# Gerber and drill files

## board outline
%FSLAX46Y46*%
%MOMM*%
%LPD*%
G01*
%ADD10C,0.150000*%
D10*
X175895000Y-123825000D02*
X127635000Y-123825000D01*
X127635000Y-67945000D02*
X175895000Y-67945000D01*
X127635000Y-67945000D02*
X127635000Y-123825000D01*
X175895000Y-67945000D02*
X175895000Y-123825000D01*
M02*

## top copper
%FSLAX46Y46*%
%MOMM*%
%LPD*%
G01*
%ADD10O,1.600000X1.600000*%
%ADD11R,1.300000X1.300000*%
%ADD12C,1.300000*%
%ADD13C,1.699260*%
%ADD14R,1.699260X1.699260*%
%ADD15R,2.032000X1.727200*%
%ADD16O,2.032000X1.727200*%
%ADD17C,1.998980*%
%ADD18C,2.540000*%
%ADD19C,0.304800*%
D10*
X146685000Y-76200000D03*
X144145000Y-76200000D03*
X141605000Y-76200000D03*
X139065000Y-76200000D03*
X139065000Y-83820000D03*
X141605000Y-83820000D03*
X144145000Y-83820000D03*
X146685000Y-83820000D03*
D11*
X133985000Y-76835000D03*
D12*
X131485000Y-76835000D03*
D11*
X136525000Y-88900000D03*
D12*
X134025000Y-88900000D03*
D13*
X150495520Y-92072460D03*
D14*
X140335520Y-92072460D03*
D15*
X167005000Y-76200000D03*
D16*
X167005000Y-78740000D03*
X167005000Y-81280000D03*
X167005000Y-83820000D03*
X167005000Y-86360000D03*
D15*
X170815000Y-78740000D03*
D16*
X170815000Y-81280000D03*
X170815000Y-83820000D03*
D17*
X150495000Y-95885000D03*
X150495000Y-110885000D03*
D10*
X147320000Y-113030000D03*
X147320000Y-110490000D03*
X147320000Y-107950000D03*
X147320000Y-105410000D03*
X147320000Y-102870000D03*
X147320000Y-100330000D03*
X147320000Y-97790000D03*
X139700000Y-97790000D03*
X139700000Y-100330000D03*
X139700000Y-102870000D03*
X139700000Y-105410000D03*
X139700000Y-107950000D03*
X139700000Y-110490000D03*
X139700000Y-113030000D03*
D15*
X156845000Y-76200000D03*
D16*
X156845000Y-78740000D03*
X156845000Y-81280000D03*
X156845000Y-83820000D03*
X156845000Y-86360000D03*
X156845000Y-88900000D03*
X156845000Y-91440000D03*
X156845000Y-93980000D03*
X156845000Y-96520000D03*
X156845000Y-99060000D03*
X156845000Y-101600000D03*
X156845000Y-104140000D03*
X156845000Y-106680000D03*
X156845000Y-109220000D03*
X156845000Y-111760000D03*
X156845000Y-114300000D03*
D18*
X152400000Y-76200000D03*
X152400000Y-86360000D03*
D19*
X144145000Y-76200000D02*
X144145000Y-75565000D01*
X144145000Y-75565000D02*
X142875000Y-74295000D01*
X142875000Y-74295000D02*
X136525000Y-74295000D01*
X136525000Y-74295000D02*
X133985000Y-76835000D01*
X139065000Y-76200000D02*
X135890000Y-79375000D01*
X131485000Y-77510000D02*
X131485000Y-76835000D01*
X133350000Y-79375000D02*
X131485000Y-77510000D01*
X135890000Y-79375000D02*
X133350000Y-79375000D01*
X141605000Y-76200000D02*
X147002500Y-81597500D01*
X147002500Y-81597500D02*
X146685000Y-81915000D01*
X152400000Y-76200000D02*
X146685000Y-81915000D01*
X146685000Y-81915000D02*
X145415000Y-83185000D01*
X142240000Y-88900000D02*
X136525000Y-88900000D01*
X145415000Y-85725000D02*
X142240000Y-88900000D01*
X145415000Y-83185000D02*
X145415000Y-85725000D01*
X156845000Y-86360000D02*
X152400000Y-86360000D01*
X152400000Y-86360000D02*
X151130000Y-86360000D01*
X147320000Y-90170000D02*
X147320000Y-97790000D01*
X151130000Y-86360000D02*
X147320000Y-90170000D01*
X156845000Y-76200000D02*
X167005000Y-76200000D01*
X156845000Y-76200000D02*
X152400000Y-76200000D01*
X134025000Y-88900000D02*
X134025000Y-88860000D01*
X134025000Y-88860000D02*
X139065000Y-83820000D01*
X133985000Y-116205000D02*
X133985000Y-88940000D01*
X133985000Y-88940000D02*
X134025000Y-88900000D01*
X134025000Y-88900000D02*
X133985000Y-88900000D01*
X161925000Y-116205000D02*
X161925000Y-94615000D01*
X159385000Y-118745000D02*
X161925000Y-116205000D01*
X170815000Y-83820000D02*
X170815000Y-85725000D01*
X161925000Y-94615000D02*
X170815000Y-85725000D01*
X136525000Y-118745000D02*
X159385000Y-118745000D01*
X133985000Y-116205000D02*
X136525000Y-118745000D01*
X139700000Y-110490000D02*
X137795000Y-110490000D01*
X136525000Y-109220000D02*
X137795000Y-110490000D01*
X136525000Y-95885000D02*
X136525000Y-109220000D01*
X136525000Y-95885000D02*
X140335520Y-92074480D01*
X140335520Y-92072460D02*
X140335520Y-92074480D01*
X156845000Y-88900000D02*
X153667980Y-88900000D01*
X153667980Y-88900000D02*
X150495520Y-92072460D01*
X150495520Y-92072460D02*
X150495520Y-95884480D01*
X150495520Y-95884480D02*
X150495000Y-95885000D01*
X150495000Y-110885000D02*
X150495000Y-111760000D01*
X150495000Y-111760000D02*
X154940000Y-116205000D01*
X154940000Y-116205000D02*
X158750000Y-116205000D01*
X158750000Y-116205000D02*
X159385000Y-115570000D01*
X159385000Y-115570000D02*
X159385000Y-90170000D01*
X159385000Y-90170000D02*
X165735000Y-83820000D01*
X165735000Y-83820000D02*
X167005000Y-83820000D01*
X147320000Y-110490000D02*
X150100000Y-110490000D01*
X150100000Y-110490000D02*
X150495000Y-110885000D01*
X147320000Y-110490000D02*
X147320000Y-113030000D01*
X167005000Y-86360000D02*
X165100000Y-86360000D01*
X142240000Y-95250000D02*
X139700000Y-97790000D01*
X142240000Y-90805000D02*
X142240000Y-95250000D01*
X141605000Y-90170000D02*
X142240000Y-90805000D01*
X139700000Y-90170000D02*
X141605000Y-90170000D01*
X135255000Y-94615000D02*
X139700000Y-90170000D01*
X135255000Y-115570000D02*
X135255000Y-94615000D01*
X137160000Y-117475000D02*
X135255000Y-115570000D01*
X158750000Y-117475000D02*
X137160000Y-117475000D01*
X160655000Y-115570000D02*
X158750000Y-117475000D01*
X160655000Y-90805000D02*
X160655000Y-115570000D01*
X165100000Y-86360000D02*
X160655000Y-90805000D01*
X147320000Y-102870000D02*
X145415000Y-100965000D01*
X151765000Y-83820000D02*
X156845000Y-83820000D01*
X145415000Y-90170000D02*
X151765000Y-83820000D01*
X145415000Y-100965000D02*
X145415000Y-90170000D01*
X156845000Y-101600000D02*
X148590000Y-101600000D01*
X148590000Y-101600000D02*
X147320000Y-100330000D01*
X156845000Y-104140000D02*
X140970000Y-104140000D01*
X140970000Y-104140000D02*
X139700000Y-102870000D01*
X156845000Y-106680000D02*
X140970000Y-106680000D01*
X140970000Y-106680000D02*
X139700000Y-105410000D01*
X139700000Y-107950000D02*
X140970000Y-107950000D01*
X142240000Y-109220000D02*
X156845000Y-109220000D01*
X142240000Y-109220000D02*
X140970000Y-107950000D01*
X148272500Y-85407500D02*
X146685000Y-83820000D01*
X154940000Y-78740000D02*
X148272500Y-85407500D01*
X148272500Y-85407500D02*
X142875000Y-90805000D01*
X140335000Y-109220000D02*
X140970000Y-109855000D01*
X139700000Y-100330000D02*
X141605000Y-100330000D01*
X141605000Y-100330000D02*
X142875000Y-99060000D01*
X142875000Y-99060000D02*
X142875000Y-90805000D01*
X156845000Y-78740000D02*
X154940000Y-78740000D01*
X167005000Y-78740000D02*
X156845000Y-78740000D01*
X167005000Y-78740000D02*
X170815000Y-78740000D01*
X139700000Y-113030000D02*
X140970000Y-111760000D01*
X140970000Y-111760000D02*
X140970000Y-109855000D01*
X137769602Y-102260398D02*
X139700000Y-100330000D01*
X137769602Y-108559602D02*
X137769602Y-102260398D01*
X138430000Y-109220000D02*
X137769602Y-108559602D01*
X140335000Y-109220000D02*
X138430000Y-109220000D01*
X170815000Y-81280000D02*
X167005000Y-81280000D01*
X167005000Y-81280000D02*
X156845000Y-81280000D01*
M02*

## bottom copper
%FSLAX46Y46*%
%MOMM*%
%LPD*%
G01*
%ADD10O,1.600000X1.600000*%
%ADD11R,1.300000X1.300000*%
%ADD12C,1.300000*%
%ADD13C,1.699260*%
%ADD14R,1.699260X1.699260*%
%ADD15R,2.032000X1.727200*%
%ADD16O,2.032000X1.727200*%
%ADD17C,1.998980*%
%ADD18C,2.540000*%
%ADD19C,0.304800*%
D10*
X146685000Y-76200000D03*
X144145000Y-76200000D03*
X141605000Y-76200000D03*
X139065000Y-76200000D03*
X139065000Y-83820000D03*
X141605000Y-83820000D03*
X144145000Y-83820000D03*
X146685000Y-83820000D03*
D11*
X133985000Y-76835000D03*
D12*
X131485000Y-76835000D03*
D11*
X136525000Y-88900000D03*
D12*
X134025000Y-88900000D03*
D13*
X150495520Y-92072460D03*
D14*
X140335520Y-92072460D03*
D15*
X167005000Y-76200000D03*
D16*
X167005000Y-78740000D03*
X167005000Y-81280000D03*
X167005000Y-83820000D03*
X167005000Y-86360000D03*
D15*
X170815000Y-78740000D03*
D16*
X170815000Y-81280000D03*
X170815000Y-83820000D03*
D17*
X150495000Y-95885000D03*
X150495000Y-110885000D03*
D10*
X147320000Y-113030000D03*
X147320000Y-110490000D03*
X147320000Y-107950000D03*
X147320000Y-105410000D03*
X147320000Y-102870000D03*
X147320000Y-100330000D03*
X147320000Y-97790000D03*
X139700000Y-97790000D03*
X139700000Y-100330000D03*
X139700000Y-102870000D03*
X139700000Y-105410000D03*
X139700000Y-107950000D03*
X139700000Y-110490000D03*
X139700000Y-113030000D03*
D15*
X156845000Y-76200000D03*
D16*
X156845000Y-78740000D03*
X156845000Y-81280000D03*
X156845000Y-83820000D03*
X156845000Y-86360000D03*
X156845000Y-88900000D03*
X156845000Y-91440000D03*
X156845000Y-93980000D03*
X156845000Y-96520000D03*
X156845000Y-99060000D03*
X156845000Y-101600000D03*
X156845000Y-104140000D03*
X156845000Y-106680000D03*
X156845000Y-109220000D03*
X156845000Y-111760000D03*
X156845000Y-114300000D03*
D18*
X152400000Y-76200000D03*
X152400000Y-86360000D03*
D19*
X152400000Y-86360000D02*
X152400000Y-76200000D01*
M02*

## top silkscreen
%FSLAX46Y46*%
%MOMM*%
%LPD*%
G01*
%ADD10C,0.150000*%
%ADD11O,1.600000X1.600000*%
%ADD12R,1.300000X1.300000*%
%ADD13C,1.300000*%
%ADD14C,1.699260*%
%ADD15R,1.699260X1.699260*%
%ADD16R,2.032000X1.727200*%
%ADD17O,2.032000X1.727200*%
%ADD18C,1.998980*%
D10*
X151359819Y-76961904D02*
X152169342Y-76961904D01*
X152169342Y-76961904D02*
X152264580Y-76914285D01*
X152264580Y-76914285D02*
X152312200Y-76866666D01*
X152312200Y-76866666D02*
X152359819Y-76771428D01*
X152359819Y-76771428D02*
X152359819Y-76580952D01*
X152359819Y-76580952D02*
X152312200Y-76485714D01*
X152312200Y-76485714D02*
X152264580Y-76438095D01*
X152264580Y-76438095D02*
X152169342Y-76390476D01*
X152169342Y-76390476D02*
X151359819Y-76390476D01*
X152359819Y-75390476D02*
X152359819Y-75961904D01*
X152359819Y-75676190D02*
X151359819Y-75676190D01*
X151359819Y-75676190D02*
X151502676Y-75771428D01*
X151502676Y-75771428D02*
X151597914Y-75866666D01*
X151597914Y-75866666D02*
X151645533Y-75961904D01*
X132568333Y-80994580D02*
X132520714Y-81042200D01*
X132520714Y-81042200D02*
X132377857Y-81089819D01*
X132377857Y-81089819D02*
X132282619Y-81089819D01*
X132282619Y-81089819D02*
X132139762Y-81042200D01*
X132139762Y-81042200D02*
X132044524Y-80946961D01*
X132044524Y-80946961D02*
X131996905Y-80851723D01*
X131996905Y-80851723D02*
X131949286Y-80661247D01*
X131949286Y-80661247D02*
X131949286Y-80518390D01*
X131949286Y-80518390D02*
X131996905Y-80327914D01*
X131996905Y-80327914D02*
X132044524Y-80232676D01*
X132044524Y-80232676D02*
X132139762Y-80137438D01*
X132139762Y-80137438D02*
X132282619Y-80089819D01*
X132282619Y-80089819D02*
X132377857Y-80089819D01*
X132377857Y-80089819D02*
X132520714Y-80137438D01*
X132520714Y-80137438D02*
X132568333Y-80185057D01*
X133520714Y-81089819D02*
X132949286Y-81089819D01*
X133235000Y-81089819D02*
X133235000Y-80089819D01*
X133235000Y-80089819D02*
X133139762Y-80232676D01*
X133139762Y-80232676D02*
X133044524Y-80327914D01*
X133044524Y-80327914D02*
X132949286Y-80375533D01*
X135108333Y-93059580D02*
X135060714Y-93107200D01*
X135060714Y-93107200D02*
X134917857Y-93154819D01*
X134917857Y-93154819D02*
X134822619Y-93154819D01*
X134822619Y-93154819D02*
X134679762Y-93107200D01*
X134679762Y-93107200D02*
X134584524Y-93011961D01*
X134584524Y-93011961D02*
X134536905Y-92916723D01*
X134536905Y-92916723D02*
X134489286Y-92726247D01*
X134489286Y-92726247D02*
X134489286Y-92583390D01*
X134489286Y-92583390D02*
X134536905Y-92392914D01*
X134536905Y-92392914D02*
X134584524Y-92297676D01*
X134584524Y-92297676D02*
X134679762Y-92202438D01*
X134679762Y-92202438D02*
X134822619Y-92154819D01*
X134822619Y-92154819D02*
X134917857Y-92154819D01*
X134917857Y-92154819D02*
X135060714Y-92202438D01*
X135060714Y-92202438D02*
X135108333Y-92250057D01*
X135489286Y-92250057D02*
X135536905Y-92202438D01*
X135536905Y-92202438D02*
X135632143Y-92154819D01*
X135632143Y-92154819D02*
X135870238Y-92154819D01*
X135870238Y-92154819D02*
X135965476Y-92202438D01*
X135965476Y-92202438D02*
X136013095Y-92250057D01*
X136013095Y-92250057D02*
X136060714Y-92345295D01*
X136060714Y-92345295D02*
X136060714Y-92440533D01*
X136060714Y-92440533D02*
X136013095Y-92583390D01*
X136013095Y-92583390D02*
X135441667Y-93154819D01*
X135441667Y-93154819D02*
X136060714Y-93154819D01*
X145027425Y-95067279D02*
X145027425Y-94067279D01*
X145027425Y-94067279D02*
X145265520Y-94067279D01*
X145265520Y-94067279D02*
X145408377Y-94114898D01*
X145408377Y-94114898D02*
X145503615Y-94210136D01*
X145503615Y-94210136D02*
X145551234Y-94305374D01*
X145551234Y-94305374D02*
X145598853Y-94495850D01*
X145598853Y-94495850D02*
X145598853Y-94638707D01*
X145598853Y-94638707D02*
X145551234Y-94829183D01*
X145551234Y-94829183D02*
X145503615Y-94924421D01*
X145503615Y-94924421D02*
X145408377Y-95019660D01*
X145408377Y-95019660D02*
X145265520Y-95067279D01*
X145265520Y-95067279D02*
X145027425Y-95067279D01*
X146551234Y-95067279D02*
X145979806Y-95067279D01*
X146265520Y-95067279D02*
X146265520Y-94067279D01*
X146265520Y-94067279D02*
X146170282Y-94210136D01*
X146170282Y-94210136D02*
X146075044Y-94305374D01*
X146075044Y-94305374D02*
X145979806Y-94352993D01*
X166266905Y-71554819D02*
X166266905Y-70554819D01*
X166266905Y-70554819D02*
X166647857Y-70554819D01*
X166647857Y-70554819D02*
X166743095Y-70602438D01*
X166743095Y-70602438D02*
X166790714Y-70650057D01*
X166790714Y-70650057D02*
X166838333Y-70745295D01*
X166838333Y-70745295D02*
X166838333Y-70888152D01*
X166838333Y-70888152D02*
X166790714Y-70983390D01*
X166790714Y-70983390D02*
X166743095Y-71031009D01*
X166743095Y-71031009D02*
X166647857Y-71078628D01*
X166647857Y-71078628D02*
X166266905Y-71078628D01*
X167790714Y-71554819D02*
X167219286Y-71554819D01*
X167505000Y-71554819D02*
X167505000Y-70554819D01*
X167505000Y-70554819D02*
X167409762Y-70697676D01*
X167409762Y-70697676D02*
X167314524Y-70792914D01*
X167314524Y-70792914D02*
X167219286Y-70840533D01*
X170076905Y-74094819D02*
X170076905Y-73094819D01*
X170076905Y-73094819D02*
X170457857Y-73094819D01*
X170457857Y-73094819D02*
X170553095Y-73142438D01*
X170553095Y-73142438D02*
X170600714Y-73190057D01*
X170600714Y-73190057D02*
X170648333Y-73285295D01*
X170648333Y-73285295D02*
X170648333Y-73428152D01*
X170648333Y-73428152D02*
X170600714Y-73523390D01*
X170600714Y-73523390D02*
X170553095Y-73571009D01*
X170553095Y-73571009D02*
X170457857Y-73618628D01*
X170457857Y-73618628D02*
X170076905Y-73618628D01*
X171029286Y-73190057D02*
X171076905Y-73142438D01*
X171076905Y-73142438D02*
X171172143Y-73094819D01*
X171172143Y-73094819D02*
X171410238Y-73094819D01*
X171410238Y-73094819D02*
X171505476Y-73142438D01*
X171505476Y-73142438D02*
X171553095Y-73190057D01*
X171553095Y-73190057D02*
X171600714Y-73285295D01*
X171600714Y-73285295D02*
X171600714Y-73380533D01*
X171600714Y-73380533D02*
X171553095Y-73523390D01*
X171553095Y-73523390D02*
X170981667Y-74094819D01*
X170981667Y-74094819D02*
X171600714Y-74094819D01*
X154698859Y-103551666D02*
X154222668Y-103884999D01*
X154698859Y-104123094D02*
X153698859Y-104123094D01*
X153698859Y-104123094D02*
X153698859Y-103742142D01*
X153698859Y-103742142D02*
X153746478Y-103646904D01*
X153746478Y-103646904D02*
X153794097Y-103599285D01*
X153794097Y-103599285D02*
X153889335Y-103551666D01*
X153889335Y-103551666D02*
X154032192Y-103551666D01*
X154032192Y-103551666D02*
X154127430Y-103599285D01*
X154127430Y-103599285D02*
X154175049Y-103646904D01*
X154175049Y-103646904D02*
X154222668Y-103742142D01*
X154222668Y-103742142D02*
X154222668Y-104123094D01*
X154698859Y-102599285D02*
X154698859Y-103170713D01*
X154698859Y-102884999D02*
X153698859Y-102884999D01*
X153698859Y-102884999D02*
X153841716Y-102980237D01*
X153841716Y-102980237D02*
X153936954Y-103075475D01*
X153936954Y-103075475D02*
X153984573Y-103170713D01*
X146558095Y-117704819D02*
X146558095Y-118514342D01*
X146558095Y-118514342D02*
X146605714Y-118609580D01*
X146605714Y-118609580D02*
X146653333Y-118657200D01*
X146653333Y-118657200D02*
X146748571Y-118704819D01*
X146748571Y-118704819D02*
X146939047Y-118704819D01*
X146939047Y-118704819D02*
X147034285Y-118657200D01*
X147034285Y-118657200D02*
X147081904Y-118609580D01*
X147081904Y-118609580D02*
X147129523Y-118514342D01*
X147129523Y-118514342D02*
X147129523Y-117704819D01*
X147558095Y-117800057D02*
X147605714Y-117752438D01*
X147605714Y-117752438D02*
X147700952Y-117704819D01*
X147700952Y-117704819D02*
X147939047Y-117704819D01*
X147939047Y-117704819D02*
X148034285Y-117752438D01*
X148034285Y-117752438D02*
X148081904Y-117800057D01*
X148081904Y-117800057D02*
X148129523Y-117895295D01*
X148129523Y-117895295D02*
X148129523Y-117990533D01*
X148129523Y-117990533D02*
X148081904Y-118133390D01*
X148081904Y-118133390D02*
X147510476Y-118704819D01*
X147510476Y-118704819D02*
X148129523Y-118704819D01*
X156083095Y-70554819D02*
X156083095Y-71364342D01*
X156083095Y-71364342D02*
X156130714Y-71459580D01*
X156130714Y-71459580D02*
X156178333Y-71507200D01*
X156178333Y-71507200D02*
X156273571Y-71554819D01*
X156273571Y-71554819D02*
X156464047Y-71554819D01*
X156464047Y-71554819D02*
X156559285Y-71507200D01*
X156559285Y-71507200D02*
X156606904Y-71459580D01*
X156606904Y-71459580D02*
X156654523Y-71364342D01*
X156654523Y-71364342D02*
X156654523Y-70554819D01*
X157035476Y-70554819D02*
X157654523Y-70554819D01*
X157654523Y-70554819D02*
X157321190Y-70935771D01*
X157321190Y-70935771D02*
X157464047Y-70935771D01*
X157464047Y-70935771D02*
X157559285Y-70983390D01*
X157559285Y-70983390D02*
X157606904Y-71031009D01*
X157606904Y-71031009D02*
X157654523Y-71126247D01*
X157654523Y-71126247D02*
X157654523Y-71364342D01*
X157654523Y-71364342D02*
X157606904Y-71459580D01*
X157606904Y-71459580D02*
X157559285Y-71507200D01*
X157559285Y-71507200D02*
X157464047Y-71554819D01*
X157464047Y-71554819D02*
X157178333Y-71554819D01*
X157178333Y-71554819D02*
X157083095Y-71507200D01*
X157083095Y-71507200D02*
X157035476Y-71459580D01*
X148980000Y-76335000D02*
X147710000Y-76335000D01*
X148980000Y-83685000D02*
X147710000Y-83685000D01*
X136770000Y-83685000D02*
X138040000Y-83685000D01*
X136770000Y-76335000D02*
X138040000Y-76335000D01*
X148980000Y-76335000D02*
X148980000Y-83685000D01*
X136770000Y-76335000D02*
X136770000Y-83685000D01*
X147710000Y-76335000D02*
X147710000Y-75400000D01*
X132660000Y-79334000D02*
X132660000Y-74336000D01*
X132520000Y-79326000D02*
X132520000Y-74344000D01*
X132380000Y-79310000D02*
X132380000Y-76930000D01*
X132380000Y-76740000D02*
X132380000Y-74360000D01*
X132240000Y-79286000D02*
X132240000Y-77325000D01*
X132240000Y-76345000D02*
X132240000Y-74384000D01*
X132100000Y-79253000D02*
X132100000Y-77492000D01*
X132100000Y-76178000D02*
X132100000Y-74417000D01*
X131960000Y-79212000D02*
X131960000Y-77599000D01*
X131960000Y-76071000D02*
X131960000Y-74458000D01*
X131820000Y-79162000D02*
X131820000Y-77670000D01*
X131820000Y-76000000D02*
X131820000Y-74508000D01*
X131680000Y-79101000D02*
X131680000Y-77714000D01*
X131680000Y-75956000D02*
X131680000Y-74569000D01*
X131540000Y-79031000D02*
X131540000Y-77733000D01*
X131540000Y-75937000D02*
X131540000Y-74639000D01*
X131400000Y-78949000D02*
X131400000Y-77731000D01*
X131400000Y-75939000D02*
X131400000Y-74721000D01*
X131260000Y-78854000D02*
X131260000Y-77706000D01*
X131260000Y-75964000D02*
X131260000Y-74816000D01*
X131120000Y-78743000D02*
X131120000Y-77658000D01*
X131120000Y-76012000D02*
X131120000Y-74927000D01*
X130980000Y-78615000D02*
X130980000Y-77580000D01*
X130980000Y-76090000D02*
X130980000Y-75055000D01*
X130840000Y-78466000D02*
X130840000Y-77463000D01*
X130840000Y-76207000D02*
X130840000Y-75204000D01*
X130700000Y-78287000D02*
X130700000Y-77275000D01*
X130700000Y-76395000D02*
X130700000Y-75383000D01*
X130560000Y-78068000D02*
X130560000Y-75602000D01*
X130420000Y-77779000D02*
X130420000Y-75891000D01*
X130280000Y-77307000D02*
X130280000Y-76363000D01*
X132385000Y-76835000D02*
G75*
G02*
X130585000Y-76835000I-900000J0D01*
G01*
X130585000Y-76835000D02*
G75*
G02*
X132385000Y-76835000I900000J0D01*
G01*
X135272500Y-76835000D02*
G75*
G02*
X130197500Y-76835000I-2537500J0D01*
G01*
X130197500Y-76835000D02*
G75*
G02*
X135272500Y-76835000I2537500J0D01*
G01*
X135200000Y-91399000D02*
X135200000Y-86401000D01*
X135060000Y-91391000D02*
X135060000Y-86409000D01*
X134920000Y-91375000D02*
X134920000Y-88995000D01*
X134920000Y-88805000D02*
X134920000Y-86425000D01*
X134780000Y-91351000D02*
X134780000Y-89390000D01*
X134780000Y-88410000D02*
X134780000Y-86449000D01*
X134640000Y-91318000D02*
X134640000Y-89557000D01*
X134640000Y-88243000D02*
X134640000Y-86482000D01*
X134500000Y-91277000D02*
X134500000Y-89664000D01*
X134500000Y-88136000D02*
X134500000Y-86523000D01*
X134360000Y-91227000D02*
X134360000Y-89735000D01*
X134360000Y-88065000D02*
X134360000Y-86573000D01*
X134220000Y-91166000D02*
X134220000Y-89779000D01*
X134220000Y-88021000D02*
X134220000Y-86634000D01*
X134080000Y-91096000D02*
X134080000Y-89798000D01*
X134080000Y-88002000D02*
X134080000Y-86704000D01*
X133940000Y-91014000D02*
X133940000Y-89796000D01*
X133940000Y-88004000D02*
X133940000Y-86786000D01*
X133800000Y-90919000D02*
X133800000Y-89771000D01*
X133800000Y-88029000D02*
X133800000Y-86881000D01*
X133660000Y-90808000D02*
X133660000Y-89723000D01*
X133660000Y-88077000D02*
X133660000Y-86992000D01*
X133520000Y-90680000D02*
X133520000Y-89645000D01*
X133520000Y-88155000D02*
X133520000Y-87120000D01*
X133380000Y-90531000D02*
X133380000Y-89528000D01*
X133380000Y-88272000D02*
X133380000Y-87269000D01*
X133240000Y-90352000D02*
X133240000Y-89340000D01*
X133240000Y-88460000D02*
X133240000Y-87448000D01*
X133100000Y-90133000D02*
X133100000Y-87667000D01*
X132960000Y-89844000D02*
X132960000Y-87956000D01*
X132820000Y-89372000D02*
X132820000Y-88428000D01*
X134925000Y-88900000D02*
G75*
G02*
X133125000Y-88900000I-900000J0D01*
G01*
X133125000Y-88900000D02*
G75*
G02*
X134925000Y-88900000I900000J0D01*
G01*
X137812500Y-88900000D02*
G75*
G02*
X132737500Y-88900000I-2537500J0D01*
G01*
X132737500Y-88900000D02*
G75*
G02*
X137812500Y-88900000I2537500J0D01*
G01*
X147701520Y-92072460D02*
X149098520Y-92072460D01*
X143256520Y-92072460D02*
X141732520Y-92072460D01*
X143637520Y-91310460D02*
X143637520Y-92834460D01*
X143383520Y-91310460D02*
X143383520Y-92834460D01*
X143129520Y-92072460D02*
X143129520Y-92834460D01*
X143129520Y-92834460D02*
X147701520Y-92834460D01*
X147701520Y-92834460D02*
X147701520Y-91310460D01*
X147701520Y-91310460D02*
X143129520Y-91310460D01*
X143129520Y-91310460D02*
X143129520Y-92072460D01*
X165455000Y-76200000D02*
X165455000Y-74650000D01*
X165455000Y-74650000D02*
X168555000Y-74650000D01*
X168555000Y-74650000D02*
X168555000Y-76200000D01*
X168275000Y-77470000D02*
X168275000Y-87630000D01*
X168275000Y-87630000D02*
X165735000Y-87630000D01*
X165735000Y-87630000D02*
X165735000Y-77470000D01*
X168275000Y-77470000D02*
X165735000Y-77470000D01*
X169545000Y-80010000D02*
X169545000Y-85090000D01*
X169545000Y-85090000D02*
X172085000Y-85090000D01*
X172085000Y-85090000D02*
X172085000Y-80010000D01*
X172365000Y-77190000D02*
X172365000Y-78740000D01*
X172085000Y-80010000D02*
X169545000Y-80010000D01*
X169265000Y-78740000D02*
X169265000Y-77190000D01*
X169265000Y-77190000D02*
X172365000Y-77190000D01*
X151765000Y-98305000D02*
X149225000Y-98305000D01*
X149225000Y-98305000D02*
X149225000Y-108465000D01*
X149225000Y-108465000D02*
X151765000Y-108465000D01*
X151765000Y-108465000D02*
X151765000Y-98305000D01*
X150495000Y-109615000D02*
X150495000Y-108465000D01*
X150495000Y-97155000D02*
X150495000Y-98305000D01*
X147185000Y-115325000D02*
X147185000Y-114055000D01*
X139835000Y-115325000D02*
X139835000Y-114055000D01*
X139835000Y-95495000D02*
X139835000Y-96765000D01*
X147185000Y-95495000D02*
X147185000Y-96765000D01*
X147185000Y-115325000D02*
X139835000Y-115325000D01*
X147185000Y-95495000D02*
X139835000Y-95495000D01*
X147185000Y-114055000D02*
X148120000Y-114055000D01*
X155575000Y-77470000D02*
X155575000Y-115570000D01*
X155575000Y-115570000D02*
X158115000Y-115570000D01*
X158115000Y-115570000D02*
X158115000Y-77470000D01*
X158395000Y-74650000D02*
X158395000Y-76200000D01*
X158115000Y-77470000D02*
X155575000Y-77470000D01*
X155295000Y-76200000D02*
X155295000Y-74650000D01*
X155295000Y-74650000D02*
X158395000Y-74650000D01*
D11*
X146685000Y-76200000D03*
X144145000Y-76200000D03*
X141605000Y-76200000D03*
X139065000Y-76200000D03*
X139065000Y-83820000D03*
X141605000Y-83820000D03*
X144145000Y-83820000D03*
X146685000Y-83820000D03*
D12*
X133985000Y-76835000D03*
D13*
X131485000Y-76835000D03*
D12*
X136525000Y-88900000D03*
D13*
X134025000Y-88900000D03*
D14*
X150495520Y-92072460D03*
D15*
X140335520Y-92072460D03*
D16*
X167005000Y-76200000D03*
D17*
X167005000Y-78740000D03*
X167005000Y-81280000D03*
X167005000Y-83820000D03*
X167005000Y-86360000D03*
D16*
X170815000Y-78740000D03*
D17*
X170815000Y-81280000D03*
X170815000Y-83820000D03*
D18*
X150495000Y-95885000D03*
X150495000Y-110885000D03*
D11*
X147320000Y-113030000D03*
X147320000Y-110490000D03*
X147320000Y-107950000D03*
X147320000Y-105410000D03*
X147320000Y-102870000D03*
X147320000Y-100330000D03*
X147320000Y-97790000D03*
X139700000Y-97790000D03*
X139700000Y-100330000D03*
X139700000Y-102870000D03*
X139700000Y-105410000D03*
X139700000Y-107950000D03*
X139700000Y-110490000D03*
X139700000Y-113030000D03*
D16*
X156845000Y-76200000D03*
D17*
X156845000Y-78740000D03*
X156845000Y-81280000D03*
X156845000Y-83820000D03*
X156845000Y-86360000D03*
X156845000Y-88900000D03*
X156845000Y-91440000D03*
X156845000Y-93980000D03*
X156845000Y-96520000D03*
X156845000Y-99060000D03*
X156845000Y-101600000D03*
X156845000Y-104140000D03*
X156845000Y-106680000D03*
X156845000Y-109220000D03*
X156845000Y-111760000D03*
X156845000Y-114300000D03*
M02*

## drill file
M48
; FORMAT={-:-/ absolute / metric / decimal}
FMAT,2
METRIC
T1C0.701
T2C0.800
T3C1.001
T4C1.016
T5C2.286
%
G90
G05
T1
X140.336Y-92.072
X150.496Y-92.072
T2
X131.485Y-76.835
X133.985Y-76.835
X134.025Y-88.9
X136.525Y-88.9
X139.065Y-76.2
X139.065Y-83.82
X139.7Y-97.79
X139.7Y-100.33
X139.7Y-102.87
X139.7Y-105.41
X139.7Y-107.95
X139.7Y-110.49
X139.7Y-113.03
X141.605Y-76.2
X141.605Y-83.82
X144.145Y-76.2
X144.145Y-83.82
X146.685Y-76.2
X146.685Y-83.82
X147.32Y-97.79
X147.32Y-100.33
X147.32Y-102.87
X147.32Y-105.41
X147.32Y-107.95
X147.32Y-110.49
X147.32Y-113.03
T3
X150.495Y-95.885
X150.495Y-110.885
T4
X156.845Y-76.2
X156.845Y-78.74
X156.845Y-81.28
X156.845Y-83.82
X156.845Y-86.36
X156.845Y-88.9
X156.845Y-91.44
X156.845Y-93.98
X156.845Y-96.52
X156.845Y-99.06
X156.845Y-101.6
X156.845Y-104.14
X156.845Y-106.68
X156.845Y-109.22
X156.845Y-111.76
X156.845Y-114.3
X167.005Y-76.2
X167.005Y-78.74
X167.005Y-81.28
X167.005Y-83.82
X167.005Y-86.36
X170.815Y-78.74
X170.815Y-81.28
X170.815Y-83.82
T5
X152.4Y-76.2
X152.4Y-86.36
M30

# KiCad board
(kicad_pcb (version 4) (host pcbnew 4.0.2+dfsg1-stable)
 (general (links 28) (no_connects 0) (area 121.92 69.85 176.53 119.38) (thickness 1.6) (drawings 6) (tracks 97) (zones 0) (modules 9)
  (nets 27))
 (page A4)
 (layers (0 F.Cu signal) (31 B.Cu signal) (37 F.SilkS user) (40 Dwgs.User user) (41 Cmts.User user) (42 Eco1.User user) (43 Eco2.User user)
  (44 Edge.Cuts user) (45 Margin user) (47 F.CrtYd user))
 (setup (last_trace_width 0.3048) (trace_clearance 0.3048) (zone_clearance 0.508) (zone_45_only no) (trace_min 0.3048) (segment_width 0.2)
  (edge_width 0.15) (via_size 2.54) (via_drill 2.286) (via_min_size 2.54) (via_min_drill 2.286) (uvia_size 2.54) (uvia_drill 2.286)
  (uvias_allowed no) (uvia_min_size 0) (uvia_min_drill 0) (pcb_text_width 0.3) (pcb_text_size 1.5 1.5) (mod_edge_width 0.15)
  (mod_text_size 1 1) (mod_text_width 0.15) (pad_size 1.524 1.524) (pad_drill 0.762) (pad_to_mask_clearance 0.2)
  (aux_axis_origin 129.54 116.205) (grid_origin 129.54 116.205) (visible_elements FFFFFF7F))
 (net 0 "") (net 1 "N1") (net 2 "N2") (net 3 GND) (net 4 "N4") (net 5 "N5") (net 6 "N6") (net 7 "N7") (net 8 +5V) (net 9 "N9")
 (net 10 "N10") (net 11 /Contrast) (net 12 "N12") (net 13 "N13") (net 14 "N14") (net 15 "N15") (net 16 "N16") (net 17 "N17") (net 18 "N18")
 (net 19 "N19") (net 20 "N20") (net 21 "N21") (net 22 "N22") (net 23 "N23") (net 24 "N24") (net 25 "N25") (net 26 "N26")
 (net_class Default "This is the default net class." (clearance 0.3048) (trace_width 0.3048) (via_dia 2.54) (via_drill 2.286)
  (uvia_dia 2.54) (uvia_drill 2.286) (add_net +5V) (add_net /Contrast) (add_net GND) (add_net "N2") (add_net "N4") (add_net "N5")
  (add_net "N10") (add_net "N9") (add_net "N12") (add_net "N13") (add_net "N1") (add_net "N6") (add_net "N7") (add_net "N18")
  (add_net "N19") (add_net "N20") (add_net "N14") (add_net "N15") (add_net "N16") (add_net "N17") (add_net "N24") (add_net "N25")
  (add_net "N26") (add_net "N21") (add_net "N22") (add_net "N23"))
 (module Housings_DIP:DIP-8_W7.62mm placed (layer F.Cu) (at 146.685 76.2 270)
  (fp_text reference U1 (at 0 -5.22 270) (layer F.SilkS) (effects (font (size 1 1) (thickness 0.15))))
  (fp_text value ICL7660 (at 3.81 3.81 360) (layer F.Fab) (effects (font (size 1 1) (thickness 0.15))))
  (fp_line (start 0.135 -2.295) (end 0.135 -1.025) (layer F.SilkS) (width 0.15))
  (fp_line (start 7.485 -2.295) (end 7.485 -1.025) (layer F.SilkS) (width 0.15))
  (fp_line (start 7.485 9.915) (end 7.485 8.645) (layer F.SilkS) (width 0.15))
  (fp_line (start 0.135 9.915) (end 0.135 8.645) (layer F.SilkS) (width 0.15))
  (fp_line (start 0.135 -2.295) (end 7.485 -2.295) (layer F.SilkS) (width 0.15))
  (fp_line (start 0.135 9.915) (end 7.485 9.915) (layer F.SilkS) (width 0.15))
  (fp_line (start 0.135 -1.025) (end -0.8 -1.025) (layer F.SilkS) (width 0.15))
  (pad 1 thru_hole oval (at 0 0 270) (size 1.6 1.6) (drill 0.8) (layers *.Cu *.Mask F.SilkS) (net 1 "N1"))
  (pad 2 thru_hole oval (at 0 2.54 270) (size 1.6 1.6) (drill 0.8) (layers *.Cu *.Mask F.SilkS) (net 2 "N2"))
  (pad 3 thru_hole oval (at 0 5.08 270) (size 1.6 1.6) (drill 0.8) (layers *.Cu *.Mask F.SilkS) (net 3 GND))
  (pad 4 thru_hole oval (at 0 7.62 270) (size 1.6 1.6) (drill 0.8) (layers *.Cu *.Mask F.SilkS) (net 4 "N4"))
  (pad 5 thru_hole oval (at 7.62 7.62 270) (size 1.6 1.6) (drill 0.8) (layers *.Cu *.Mask F.SilkS) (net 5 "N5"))
  (pad 6 thru_hole oval (at 7.62 5.08 270) (size 1.6 1.6) (drill 0.8) (layers *.Cu *.Mask F.SilkS) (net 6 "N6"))
  (pad 7 thru_hole oval (at 7.62 2.54 270) (size 1.6 1.6) (drill 0.8) (layers *.Cu *.Mask F.SilkS) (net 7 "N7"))
  (pad 8 thru_hole oval (at 7.62 0 270) (size 1.6 1.6) (drill 0.8) (layers *.Cu *.Mask F.SilkS) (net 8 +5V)))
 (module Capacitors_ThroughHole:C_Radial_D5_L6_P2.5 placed (layer F.Cu) (at 133.985 76.835 180)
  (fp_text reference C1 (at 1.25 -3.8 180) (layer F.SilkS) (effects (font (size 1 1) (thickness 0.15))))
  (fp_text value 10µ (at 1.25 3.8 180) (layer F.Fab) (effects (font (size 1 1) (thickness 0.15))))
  (fp_line (start 1.325 -2.499) (end 1.325 2.499) (layer F.SilkS) (width 0.15))
  (fp_line (start 1.465 -2.491) (end 1.465 2.491) (layer F.SilkS) (width 0.15))
  (fp_line (start 1.605 -2.475) (end 1.605 -0.095) (layer F.SilkS) (width 0.15))
  (fp_line (start 1.605 0.095) (end 1.605 2.475) (layer F.SilkS) (width 0.15))
  (fp_line (start 1.745 -2.451) (end 1.745 -0.49) (layer F.SilkS) (width 0.15))
  (fp_line (start 1.745 0.49) (end 1.745 2.451) (layer F.SilkS) (width 0.15))
  (fp_line (start 1.885 -2.418) (end 1.885 -0.657) (layer F.SilkS) (width 0.15))
  (fp_line (start 1.885 0.657) (end 1.885 2.418) (layer F.SilkS) (width 0.15))
  (fp_line (start 2.025 -2.377) (end 2.025 -0.764) (layer F.SilkS) (width 0.15))
  (fp_line (start 2.025 0.764) (end 2.025 2.377) (layer F.SilkS) (width 0.15))
  (fp_line (start 2.165 -2.327) (end 2.165 -0.835) (layer F.SilkS) (width 0.15))
  (fp_line (start 2.165 0.835) (end 2.165 2.327) (layer F.SilkS) (width 0.15))
  (fp_line (start 2.305 -2.266) (end 2.305 -0.879) (layer F.SilkS) (width 0.15))
  (fp_line (start 2.305 0.879) (end 2.305 2.266) (layer F.SilkS) (width 0.15))
  (fp_line (start 2.445 -2.196) (end 2.445 -0.898) (layer F.SilkS) (width 0.15))
  (fp_line (start 2.445 0.898) (end 2.445 2.196) (layer F.SilkS) (width 0.15))
  (fp_line (start 2.585 -2.114) (end 2.585 -0.896) (layer F.SilkS) (width 0.15))
  (fp_line (start 2.585 0.896) (end 2.585 2.114) (layer F.SilkS) (width 0.15))
  (fp_line (start 2.725 -2.019) (end 2.725 -0.871) (layer F.SilkS) (width 0.15))
  (fp_line (start 2.725 0.871) (end 2.725 2.019) (layer F.SilkS) (width 0.15))
  (fp_line (start 2.865 -1.908) (end 2.865 -0.823) (layer F.SilkS) (width 0.15))
  (fp_line (start 2.865 0.823) (end 2.865 1.908) (layer F.SilkS) (width 0.15))
  (fp_line (start 3.005 -1.78) (end 3.005 -0.745) (layer F.SilkS) (width 0.15))
  (fp_line (start 3.005 0.745) (end 3.005 1.78) (layer F.SilkS) (width 0.15))
  (fp_line (start 3.145 -1.631) (end 3.145 -0.628) (layer F.SilkS) (width 0.15))
  (fp_line (start 3.145 0.628) (end 3.145 1.631) (layer F.SilkS) (width 0.15))
  (fp_line (start 3.285 -1.452) (end 3.285 -0.44) (layer F.SilkS) (width 0.15))
  (fp_line (start 3.285 0.44) (end 3.285 1.452) (layer F.SilkS) (width 0.15))
  (fp_line (start 3.425 -1.233) (end 3.425 1.233) (layer F.SilkS) (width 0.15))
  (fp_line (start 3.565 -0.944) (end 3.565 0.944) (layer F.SilkS) (width 0.15))
  (fp_line (start 3.705 -0.472) (end 3.705 0.472) (layer F.SilkS) (width 0.15))
  (fp_circle (center 2.5 0) (end 2.5 -0.9) (layer F.SilkS) (width 0.15))
  (fp_circle (center 1.25 0) (end 1.25 -2.5375) (layer F.SilkS) (width 0.15))
  (pad 1 thru_hole rect (at 0 0 180) (size 1.3 1.3) (drill 0.8) (layers *.Cu *.Mask F.SilkS) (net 2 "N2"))
  (pad 2 thru_hole circle (at 2.5 0 180) (size 1.3 1.3) (drill 0.8) (layers *.Cu *.Mask F.SilkS) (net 4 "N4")))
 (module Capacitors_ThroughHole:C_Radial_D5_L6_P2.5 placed (layer F.Cu) (at 136.525 88.9 180)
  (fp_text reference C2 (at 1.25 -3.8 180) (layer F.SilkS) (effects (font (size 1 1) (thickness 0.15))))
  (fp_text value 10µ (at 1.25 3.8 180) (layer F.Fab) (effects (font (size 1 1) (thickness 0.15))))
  (fp_line (start 1.325 -2.499) (end 1.325 2.499) (layer F.SilkS) (width 0.15))
  (fp_line (start 1.465 -2.491) (end 1.465 2.491) (layer F.SilkS) (width 0.15))
  (fp_line (start 1.605 -2.475) (end 1.605 -0.095) (layer F.SilkS) (width 0.15))
  (fp_line (start 1.605 0.095) (end 1.605 2.475) (layer F.SilkS) (width 0.15))
  (fp_line (start 1.745 -2.451) (end 1.745 -0.49) (layer F.SilkS) (width 0.15))
  (fp_line (start 1.745 0.49) (end 1.745 2.451) (layer F.SilkS) (width 0.15))
  (fp_line (start 1.885 -2.418) (end 1.885 -0.657) (layer F.SilkS) (width 0.15))
  (fp_line (start 1.885 0.657) (end 1.885 2.418) (layer F.SilkS) (width 0.15))
  (fp_line (start 2.025 -2.377) (end 2.025 -0.764) (layer F.SilkS) (width 0.15))
  (fp_line (start 2.025 0.764) (end 2.025 2.377) (layer F.SilkS) (width 0.15))
  (fp_line (start 2.165 -2.327) (end 2.165 -0.835) (layer F.SilkS) (width 0.15))
  (fp_line (start 2.165 0.835) (end 2.165 2.327) (layer F.SilkS) (width 0.15))
  (fp_line (start 2.305 -2.266) (end 2.305 -0.879) (layer F.SilkS) (width 0.15))
  (fp_line (start 2.305 0.879) (end 2.305 2.266) (layer F.SilkS) (width 0.15))
  (fp_line (start 2.445 -2.196) (end 2.445 -0.898) (layer F.SilkS) (width 0.15))
  (fp_line (start 2.445 0.898) (end 2.445 2.196) (layer F.SilkS) (width 0.15))
  (fp_line (start 2.585 -2.114) (end 2.585 -0.896) (layer F.SilkS) (width 0.15))
  (fp_line (start 2.585 0.896) (end 2.585 2.114) (layer F.SilkS) (width 0.15))
  (fp_line (start 2.725 -2.019) (end 2.725 -0.871) (layer F.SilkS) (width 0.15))
  (fp_line (start 2.725 0.871) (end 2.725 2.019) (layer F.SilkS) (width 0.15))
  (fp_line (start 2.865 -1.908) (end 2.865 -0.823) (layer F.SilkS) (width 0.15))
  (fp_line (start 2.865 0.823) (end 2.865 1.908) (layer F.SilkS) (width 0.15))
  (fp_line (start 3.005 -1.78) (end 3.005 -0.745) (layer F.SilkS) (width 0.15))
  (fp_line (start 3.005 0.745) (end 3.005 1.78) (layer F.SilkS) (width 0.15))
  (fp_line (start 3.145 -1.631) (end 3.145 -0.628) (layer F.SilkS) (width 0.15))
  (fp_line (start 3.145 0.628) (end 3.145 1.631) (layer F.SilkS) (width 0.15))
  (fp_line (start 3.285 -1.452) (end 3.285 -0.44) (layer F.SilkS) (width 0.15))
  (fp_line (start 3.285 0.44) (end 3.285 1.452) (layer F.SilkS) (width 0.15))
  (fp_line (start 3.425 -1.233) (end 3.425 1.233) (layer F.SilkS) (width 0.15))
  (fp_line (start 3.565 -0.944) (end 3.565 0.944) (layer F.SilkS) (width 0.15))
  (fp_line (start 3.705 -0.472) (end 3.705 0.472) (layer F.SilkS) (width 0.15))
  (fp_circle (center 2.5 0) (end 2.5 -0.9) (layer F.SilkS) (width 0.15))
  (fp_circle (center 1.25 0) (end 1.25 -2.5375) (layer F.SilkS) (width 0.15))
  (pad 1 thru_hole rect (at 0 0 180) (size 1.3 1.3) (drill 0.8) (layers *.Cu *.Mask F.SilkS) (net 3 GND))
  (pad 2 thru_hole circle (at 2.5 0 180) (size 1.3 1.3) (drill 0.8) (layers *.Cu *.Mask F.SilkS) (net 5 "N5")))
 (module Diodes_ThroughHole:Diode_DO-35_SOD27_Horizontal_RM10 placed (layer F.Cu) (at 140.335 92.075)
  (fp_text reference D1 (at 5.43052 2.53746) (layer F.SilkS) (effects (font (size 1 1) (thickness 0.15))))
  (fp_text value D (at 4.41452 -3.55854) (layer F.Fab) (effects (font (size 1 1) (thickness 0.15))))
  (fp_line (start 7.36652 -0.00254) (end 8.76352 -0.00254) (layer F.SilkS) (width 0.15))
  (fp_line (start 2.92152 -0.00254) (end 1.39752 -0.00254) (layer F.SilkS) (width 0.15))
  (fp_line (start 3.30252 -0.76454) (end 3.30252 0.75946) (layer F.SilkS) (width 0.15))
  (fp_line (start 3.04852 -0.76454) (end 3.04852 0.75946) (layer F.SilkS) (width 0.15))
  (fp_line (start 2.79452 -0.00254) (end 2.79452 0.75946) (layer F.SilkS) (width 0.15))
  (fp_line (start 2.79452 0.75946) (end 7.36652 0.75946) (layer F.SilkS) (width 0.15))
  (fp_line (start 7.36652 0.75946) (end 7.36652 -0.76454) (layer F.SilkS) (width 0.15))
  (fp_line (start 7.36652 -0.76454) (end 2.79452 -0.76454) (layer F.SilkS) (width 0.15))
  (fp_line (start 2.79452 -0.76454) (end 2.79452 -0.00254) (layer F.SilkS) (width 0.15))
  (pad 2 thru_hole circle (at 10.16052 -0.00254 180) (size 1.69926 1.69926) (drill 0.70104) (layers *.Cu *.Mask F.SilkS) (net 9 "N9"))
  (pad 1 thru_hole rect (at 0.00052 -0.00254 180) (size 1.69926 1.69926) (drill 0.70104) (layers *.Cu *.Mask F.SilkS) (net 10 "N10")))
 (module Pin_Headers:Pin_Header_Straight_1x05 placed (layer F.Cu) (at 167.005 76.2)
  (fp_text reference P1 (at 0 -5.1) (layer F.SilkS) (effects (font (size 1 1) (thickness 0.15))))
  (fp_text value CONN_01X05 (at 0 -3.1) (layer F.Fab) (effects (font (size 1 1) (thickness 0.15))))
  (fp_line (start -1.55 0) (end -1.55 -1.55) (layer F.SilkS) (width 0.15))
  (fp_line (start -1.55 -1.55) (end 1.55 -1.55) (layer F.SilkS) (width 0.15))
  (fp_line (start 1.55 -1.55) (end 1.55 0) (layer F.SilkS) (width 0.15))
  (fp_line (start 1.27 1.27) (end 1.27 11.43) (layer F.SilkS) (width 0.15))
  (fp_line (start 1.27 11.43) (end -1.27 11.43) (layer F.SilkS) (width 0.15))
  (fp_line (start -1.27 11.43) (end -1.27 1.27) (layer F.SilkS) (width 0.15))
  (fp_line (start 1.27 1.27) (end -1.27 1.27) (layer F.SilkS) (width 0.15))
  (pad 1 thru_hole rect (at 0 0) (size 2.032 1.7272) (drill 1.016) (layers *.Cu *.Mask F.SilkS) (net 3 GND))
  (pad 2 thru_hole oval (at 0 2.54) (size 2.032 1.7272) (drill 1.016) (layers *.Cu *.Mask F.SilkS) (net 8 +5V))
  (pad 3 thru_hole oval (at 0 5.08) (size 2.032 1.7272) (drill 1.016) (layers *.Cu *.Mask F.SilkS) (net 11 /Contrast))
  (pad 4 thru_hole oval (at 0 7.62) (size 2.032 1.7272) (drill 1.016) (layers *.Cu *.Mask F.SilkS) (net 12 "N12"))
  (pad 5 thru_hole oval (at 0 10.16) (size 2.032 1.7272) (drill 1.016) (layers *.Cu *.Mask F.SilkS) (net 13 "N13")))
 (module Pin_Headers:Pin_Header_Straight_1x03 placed (layer F.Cu) (at 170.815 78.74)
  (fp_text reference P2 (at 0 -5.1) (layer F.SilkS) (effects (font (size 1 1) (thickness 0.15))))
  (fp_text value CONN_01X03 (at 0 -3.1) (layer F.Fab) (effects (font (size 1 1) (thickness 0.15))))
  (fp_line (start -1.27 1.27) (end -1.27 6.35) (layer F.SilkS) (width 0.15))
  (fp_line (start -1.27 6.35) (end 1.27 6.35) (layer F.SilkS) (width 0.15))
  (fp_line (start 1.27 6.35) (end 1.27 1.27) (layer F.SilkS) (width 0.15))
  (fp_line (start 1.55 -1.55) (end 1.55 0) (layer F.SilkS) (width 0.15))
  (fp_line (start 1.27 1.27) (end -1.27 1.27) (layer F.SilkS) (width 0.15))
  (fp_line (start -1.55 0) (end -1.55 -1.55) (layer F.SilkS) (width 0.15))
  (fp_line (start -1.55 -1.55) (end 1.55 -1.55) (layer F.SilkS) (width 0.15))
  (pad 1 thru_hole rect (at 0 0) (size 2.032 1.7272) (drill 1.016) (layers *.Cu *.Mask F.SilkS) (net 8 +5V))
  (pad 2 thru_hole oval (at 0 2.54) (size 2.032 1.7272) (drill 1.016) (layers *.Cu *.Mask F.SilkS) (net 11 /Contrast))
  (pad 3 thru_hole oval (at 0 5.08) (size 2.032 1.7272) (drill 1.016) (layers *.Cu *.Mask F.SilkS) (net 5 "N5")))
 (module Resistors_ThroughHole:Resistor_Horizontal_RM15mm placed (layer F.Cu) (at 150.495 95.885 270)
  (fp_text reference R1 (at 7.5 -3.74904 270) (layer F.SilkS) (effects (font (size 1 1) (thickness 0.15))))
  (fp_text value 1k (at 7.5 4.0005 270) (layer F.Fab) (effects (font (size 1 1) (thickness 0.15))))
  (fp_line (start 2.42 -1.27) (end 2.42 1.27) (layer F.SilkS) (width 0.15))
  (fp_line (start 2.42 1.27) (end 12.58 1.27) (layer F.SilkS) (width 0.15))
  (fp_line (start 12.58 1.27) (end 12.58 -1.27) (layer F.SilkS) (width 0.15))
  (fp_line (start 12.58 -1.27) (end 2.42 -1.27) (layer F.SilkS) (width 0.15))
  (fp_line (start 13.73 0) (end 12.58 0) (layer F.SilkS) (width 0.15))
  (fp_line (start 1.27 0) (end 2.42 0) (layer F.SilkS) (width 0.15))
  (pad 1 thru_hole circle (at 0 0 270) (size 1.99898 1.99898) (drill 1.00076) (layers *.Cu *.SilkS *.Mask) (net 9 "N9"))
  (pad 2 thru_hole circle (at 15 0 270) (size 1.99898 1.99898) (drill 1.00076) (layers *.Cu *.SilkS *.Mask) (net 12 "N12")))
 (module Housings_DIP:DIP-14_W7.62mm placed (layer F.Cu) (at 147.32 113.03 180)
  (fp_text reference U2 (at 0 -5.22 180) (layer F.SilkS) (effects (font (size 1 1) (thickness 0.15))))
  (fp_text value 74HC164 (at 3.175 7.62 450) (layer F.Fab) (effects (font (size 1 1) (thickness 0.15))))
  (fp_line (start 0.135 -2.295) (end 0.135 -1.025) (layer F.SilkS) (width 0.15))
  (fp_line (start 7.485 -2.295) (end 7.485 -1.025) (layer F.SilkS) (width 0.15))
  (fp_line (start 7.485 17.535) (end 7.485 16.265) (layer F.SilkS) (width 0.15))
  (fp_line (start 0.135 17.535) (end 0.135 16.265) (layer F.SilkS) (width 0.15))
  (fp_line (start 0.135 -2.295) (end 7.485 -2.295) (layer F.SilkS) (width 0.15))
  (fp_line (start 0.135 17.535) (end 7.485 17.535) (layer F.SilkS) (width 0.15))
  (fp_line (start 0.135 -1.025) (end -0.8 -1.025) (layer F.SilkS) (width 0.15))
  (pad 1 thru_hole oval (at 0 0 180) (size 1.6 1.6) (drill 0.8) (layers *.Cu *.Mask F.SilkS) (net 12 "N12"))
  (pad 2 thru_hole oval (at 0 2.54 180) (size 1.6 1.6) (drill 0.8) (layers *.Cu *.Mask F.SilkS) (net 12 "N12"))
  (pad 3 thru_hole oval (at 0 5.08 180) (size 1.6 1.6) (drill 0.8) (layers *.Cu *.Mask F.SilkS) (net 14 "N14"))
  (pad 4 thru_hole oval (at 0 7.62 180) (size 1.6 1.6) (drill 0.8) (layers *.Cu *.Mask F.SilkS) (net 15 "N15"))
  (pad 5 thru_hole oval (at 0 10.16 180) (size 1.6 1.6) (drill 0.8) (layers *.Cu *.Mask F.SilkS) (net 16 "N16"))
  (pad 6 thru_hole oval (at 0 12.7 180) (size 1.6 1.6) (drill 0.8) (layers *.Cu *.Mask F.SilkS) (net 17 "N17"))
  (pad 7 thru_hole oval (at 0 15.24 180) (size 1.6 1.6) (drill 0.8) (layers *.Cu *.Mask F.SilkS) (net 3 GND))
  (pad 8 thru_hole oval (at 7.62 15.24 180) (size 1.6 1.6) (drill 0.8) (layers *.Cu *.Mask F.SilkS) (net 13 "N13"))
  (pad 9 thru_hole oval (at 7.62 12.7 180) (size 1.6 1.6) (drill 0.8) (layers *.Cu *.Mask F.SilkS) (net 8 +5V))
  (pad 10 thru_hole oval (at 7.62 10.16 180) (size 1.6 1.6) (drill 0.8) (layers *.Cu *.Mask F.SilkS) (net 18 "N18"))
  (pad 11 thru_hole oval (at 7.62 7.62 180) (size 1.6 1.6) (drill 0.8) (layers *.Cu *.Mask F.SilkS) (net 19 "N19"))
  (pad 12 thru_hole oval (at 7.62 5.08 180) (size 1.6 1.6) (drill 0.8) (layers *.Cu *.Mask F.SilkS) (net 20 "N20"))
  (pad 13 thru_hole oval (at 7.62 2.54 180) (size 1.6 1.6) (drill 0.8) (layers *.Cu *.Mask F.SilkS) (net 10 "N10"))
  (pad 14 thru_hole oval (at 7.62 0 180) (size 1.6 1.6) (drill 0.8) (layers *.Cu *.Mask F.SilkS) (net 8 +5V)))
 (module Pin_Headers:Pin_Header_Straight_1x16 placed (layer F.Cu) (at 156.845 76.2)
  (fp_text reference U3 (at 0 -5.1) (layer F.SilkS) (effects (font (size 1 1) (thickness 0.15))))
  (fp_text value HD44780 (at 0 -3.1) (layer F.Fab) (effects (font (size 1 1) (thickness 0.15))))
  (fp_line (start -1.27 1.27) (end -1.27 39.37) (layer F.SilkS) (width 0.15))
  (fp_line (start -1.27 39.37) (end 1.27 39.37) (layer F.SilkS) (width 0.15))
  (fp_line (start 1.27 39.37) (end 1.27 1.27) (layer F.SilkS) (width 0.15))
  (fp_line (start 1.55 -1.55) (end 1.55 0) (layer F.SilkS) (width 0.15))
  (fp_line (start 1.27 1.27) (end -1.27 1.27) (layer F.SilkS) (width 0.15))
  (fp_line (start -1.55 0) (end -1.55 -1.55) (layer F.SilkS) (width 0.15))
  (fp_line (start -1.55 -1.55) (end 1.55 -1.55) (layer F.SilkS) (width 0.15))
  (pad 1 thru_hole rect (at 0 0) (size 2.032 1.7272) (drill 1.016) (layers *.Cu *.Mask F.SilkS) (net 3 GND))
  (pad 2 thru_hole oval (at 0 2.54) (size 2.032 1.7272) (drill 1.016) (layers *.Cu *.Mask F.SilkS) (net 8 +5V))
  (pad 3 thru_hole oval (at 0 5.08) (size 2.032 1.7272) (drill 1.016) (layers *.Cu *.Mask F.SilkS) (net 11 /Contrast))
  (pad 4 thru_hole oval (at 0 7.62) (size 2.032 1.7272) (drill 1.016) (layers *.Cu *.Mask F.SilkS) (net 16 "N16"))
  (pad 5 thru_hole oval (at 0 10.16) (size 2.032 1.7272) (drill 1.016) (layers *.Cu *.Mask F.SilkS) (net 3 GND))
  (pad 6 thru_hole oval (at 0 12.7) (size 2.032 1.7272) (drill 1.016) (layers *.Cu *.Mask F.SilkS) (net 9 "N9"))
  (pad 7 thru_hole oval (at 0 15.24) (size 2.032 1.7272) (drill 1.016) (layers *.Cu *.Mask F.SilkS) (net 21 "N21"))
  (pad 8 thru_hole oval (at 0 17.78) (size 2.032 1.7272) (drill 1.016) (layers *.Cu *.Mask F.SilkS) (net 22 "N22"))
  (pad 9 thru_hole oval (at 0 20.32) (size 2.032 1.7272) (drill 1.016) (layers *.Cu *.Mask F.SilkS) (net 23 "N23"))
  (pad 10 thru_hole oval (at 0 22.86) (size 2.032 1.7272) (drill 1.016) (layers *.Cu *.Mask F.SilkS) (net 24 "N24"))
  (pad 11 thru_hole oval (at 0 25.4) (size 2.032 1.7272) (drill 1.016) (layers *.Cu *.Mask F.SilkS) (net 17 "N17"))
  (pad 12 thru_hole oval (at 0 27.94) (size 2.032 1.7272) (drill 1.016) (layers *.Cu *.Mask F.SilkS) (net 18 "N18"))
  (pad 13 thru_hole oval (at 0 30.48) (size 2.032 1.7272) (drill 1.016) (layers *.Cu *.Mask F.SilkS) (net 19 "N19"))
  (pad 14 thru_hole oval (at 0 33.02) (size 2.032 1.7272) (drill 1.016) (layers *.Cu *.Mask F.SilkS) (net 20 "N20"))
  (pad 15 thru_hole oval (at 0 35.56) (size 2.032 1.7272) (drill 1.016) (layers *.Cu *.Mask F.SilkS) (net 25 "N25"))
  (pad 16 thru_hole oval (at 0 38.1) (size 2.032 1.7272) (drill 1.016) (layers *.Cu *.Mask F.SilkS) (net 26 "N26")))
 (gr_line (start 175.895 123.825) (end 127.635 123.825) (angle 90) (layer Edge.Cuts) (width 0.15))
 (gr_line (start 127.635 67.945) (end 175.895 67.945) (angle 90) (layer Edge.Cuts) (width 0.15))
 (gr_line (start 127.635 67.945) (end 127.635 123.825) (angle 90) (layer Edge.Cuts) (width 0.15))
 (gr_line (start 175.895 67.945) (end 175.895 123.825) (angle 90) (layer Edge.Cuts) (width 0.15))
 (segment (start 144.145 76.2) (end 144.145 75.565) (width 0.3048) (layer F.Cu) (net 2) (status 30))
 (segment (start 144.145 75.565) (end 142.875 74.295) (width 0.3048) (layer F.Cu) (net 2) (status 10))
 (segment (start 142.875 74.295) (end 136.525 74.295) (width 0.3048) (layer F.Cu) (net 2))
 (segment (start 136.525 74.295) (end 133.985 76.835) (width 0.3048) (layer F.Cu) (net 2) (status 20))
 (segment (start 139.065 76.2) (end 135.89 79.375) (width 0.3048) (layer F.Cu) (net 4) (status 10))
 (segment (start 131.485 77.51) (end 131.485 76.835) (width 0.3048) (layer F.Cu) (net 4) (status 20))
 (segment (start 133.35 79.375) (end 131.485 77.51) (width 0.3048) (layer F.Cu) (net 4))
 (segment (start 135.89 79.375) (end 133.35 79.375) (width 0.3048) (layer F.Cu) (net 4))
 (segment (start 141.605 76.2) (end 147.0025 81.5975) (width 0.3048) (layer F.Cu) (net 3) (status 10))
 (segment (start 147.0025 81.5975) (end 146.685 81.915) (width 0.3048) (layer F.Cu) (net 3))
 (segment (start 152.4 76.2) (end 146.685 81.915) (width 0.3048) (layer F.Cu) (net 3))
 (segment (start 146.685 81.915) (end 145.415 83.185) (width 0.3048) (layer F.Cu) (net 3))
 (segment (start 142.24 88.9) (end 136.525 88.9) (width 0.3048) (layer F.Cu) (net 3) (status 20))
 (segment (start 145.415 85.725) (end 142.24 88.9) (width 0.3048) (layer F.Cu) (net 3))
 (segment (start 145.415 83.185) (end 145.415 85.725) (width 0.3048) (layer F.Cu) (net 3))
 (via (at 152.4 76.2) (size 2.54) (drill 2.286) (layers F.Cu B.Cu) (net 3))
 (segment (start 152.4 86.36) (end 152.4 76.2) (width 0.3048) (layer B.Cu) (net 3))
 (via (at 152.4 86.36) (size 2.54) (drill 2.286) (layers F.Cu B.Cu) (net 3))
 (segment (start 156.845 86.36) (end 152.4 86.36) (width 0.3048) (layer F.Cu) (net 3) (status 10))
 (segment (start 152.4 86.36) (end 151.13 86.36) (width 0.3048) (layer F.Cu) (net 3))
 (segment (start 147.32 90.17) (end 147.32 97.79) (width 0.3048) (layer F.Cu) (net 3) (status 20))
 (segment (start 151.13 86.36) (end 147.32 90.17) (width 0.3048) (layer F.Cu) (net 3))
 (segment (start 156.845 76.2) (end 167.005 76.2) (width 0.3048) (layer F.Cu) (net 3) (status 30))
 (segment (start 156.845 76.2) (end 152.4 76.2) (width 0.3048) (layer F.Cu) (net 3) (status 10))
 (segment (start 134.025 88.9) (end 134.025 88.86) (width 0.3048) (layer F.Cu) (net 5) (status 30))
 (segment (start 134.025 88.86) (end 139.065 83.82) (width 0.3048) (layer F.Cu) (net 5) (status 30))
 (segment (start 133.985 116.205) (end 133.985 88.94) (width 0.3048) (layer F.Cu) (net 5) (status 20))
 (segment (start 133.985 88.94) (end 134.025 88.9) (width 0.3048) (layer F.Cu) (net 5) (status 30))
 (segment (start 134.025 88.9) (end 133.985 88.9) (width 0.3048) (layer F.Cu) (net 5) (status 30))
 (segment (start 161.925 116.205) (end 161.925 94.615) (width 0.3048) (layer F.Cu) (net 5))
 (segment (start 159.385 118.745) (end 161.925 116.205) (width 0.3048) (layer F.Cu) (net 5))
 (segment (start 170.815 83.82) (end 170.815 85.725) (width 0.3048) (layer F.Cu) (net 5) (status 10))
 (segment (start 161.925 94.615) (end 170.815 85.725) (width 0.3048) (layer F.Cu) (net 5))
 (segment (start 136.525 118.745) (end 159.385 118.745) (width 0.3048) (layer F.Cu) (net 5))
 (segment (start 133.985 116.205) (end 136.525 118.745) (width 0.3048) (layer F.Cu) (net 5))
 (segment (start 139.7 110.49) (end 137.795 110.49) (width 0.3048) (layer F.Cu) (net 10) (status 10))
 (segment (start 136.525 109.22) (end 137.795 110.49) (width 0.3048) (layer F.Cu) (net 10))
 (segment (start 136.525 95.885) (end 136.525 109.22) (width 0.3048) (layer F.Cu) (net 10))
 (segment (start 136.525 95.885) (end 140.33552 92.07448) (width 0.3048) (layer F.Cu) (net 10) (status 20))
 (segment (start 140.33552 92.07246) (end 140.33552 92.07448) (width 0.3048) (layer F.Cu) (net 10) (status 30))
 (segment (start 156.845 88.9) (end 153.66798 88.9) (width 0.3048) (layer F.Cu) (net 9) (status 10))
 (segment (start 153.66798 88.9) (end 150.49552 92.07246) (width 0.3048) (layer F.Cu) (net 9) (status 20))
 (segment (start 150.49552 92.07246) (end 150.49552 95.88448) (width 0.3048) (layer F.Cu) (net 9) (status 30))
 (segment (start 150.49552 95.88448) (end 150.495 95.885) (width 0.3048) (layer F.Cu) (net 9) (status 30))
 (segment (start 150.495 110.885) (end 150.495 111.76) (width 0.3048) (layer F.Cu) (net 12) (status 80030))
 (segment (start 150.495 111.76) (end 154.94 116.205) (width 0.3048) (layer F.Cu) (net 12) (status 80010))
 (segment (start 154.94 116.205) (end 158.75 116.205) (width 0.3048) (layer F.Cu) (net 12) (status 80000))
 (segment (start 158.75 116.205) (end 159.385 115.57) (width 0.3048) (layer F.Cu) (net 12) (status 80000))
 (segment (start 159.385 115.57) (end 159.385 90.17) (width 0.3048) (layer F.Cu) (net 12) (status 80000))
 (segment (start 159.385 90.17) (end 165.735 83.82) (width 0.3048) (layer F.Cu) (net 12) (status 80000))
 (segment (start 165.735 83.82) (end 167.005 83.82) (width 0.3048) (layer F.Cu) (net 12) (status 80020))
 (segment (start 147.32 110.49) (end 150.1 110.49) (width 0.3048) (layer F.Cu) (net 12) (status 30))
 (segment (start 150.1 110.49) (end 150.495 110.885) (width 0.3048) (layer F.Cu) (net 12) (status 30))
 (segment (start 147.32 110.49) (end 147.32 113.03) (width 0.3048) (layer F.Cu) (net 12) (status 30))
 (segment (start 167.005 86.36) (end 165.1 86.36) (width 0.3048) (layer F.Cu) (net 13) (status 10))
 (segment (start 142.24 95.25) (end 139.7 97.79) (width 0.3048) (layer F.Cu) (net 13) (status 20))
 (segment (start 142.24 90.805) (end 142.24 95.25) (width 0.3048) (layer F.Cu) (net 13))
 (segment (start 141.605 90.17) (end 142.24 90.805) (width 0.3048) (layer F.Cu) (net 13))
 (segment (start 139.7 90.17) (end 141.605 90.17) (width 0.3048) (layer F.Cu) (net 13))
 (segment (start 135.255 94.615) (end 139.7 90.17) (width 0.3048) (layer F.Cu) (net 13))
 (segment (start 135.255 115.57) (end 135.255 94.615) (width 0.3048) (layer F.Cu) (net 13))
 (segment (start 137.16 117.475) (end 135.255 115.57) (width 0.3048) (layer F.Cu) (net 13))
 (segment (start 158.75 117.475) (end 137.16 117.475) (width 0.3048) (layer F.Cu) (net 13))
 (segment (start 160.655 115.57) (end 158.75 117.475) (width 0.3048) (layer F.Cu) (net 13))
 (segment (start 160.655 90.805) (end 160.655 115.57) (width 0.3048) (layer F.Cu) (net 13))
 (segment (start 165.1 86.36) (end 160.655 90.805) (width 0.3048) (layer F.Cu) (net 13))
 (segment (start 147.32 102.87) (end 145.415 100.965) (width 0.3048) (layer F.Cu) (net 16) (status 10))
 (segment (start 151.765 83.82) (end 156.845 83.82) (width 0.3048) (layer F.Cu) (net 16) (status 20))
 (segment (start 145.415 90.17) (end 151.765 83.82) (width 0.3048) (layer F.Cu) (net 16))
 (segment (start 145.415 100.965) (end 145.415 90.17) (width 0.3048) (layer F.Cu) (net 16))
 (segment (start 156.845 101.6) (end 148.59 101.6) (width 0.3048) (layer F.Cu) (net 17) (status 10))
 (segment (start 148.59 101.6) (end 147.32 100.33) (width 0.3048) (layer F.Cu) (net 17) (status 20))
 (segment (start 156.845 104.14) (end 140.97 104.14) (width 0.3048) (layer F.Cu) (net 18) (status 10))
 (segment (start 140.97 104.14) (end 139.7 102.87) (width 0.3048) (layer F.Cu) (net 18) (status 20))
 (segment (start 156.845 106.68) (end 140.97 106.68) (width 0.3048) (layer F.Cu) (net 19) (status 10))
 (segment (start 140.97 106.68) (end 139.7 105.41) (width 0.3048) (layer F.Cu) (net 19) (status 20))
 (segment (start 139.7 107.95) (end 140.97 107.95) (width 0.3048) (layer F.Cu) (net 20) (status 10))
 (segment (start 142.24 109.22) (end 156.845 109.22) (width 0.3048) (layer F.Cu) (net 20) (status 20))
 (segment (start 142.24 109.22) (end 140.97 107.95) (width 0.3048) (layer F.Cu) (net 20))
 (segment (start 148.2725 85.4075) (end 146.685 83.82) (width 0.3048) (layer F.Cu) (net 8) (status 20))
 (segment (start 154.94 78.74) (end 148.2725 85.4075) (width 0.3048) (layer F.Cu) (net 8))
 (segment (start 148.2725 85.4075) (end 142.875 90.805) (width 0.3048) (layer F.Cu) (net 8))
 (segment (start 140.335 109.22) (end 140.97 109.855) (width 0.3048) (layer F.Cu) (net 8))
 (segment (start 139.7 100.33) (end 141.605 100.33) (width 0.3048) (layer F.Cu) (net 8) (status 10))
 (segment (start 141.605 100.33) (end 142.875 99.06) (width 0.3048) (layer F.Cu) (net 8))
 (segment (start 142.875 99.06) (end 142.875 90.805) (width 0.3048) (layer F.Cu) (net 8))
 (segment (start 156.845 78.74) (end 154.94 78.74) (width 0.3048) (layer F.Cu) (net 8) (status 10))
 (segment (start 167.005 78.74) (end 156.845 78.74) (width 0.3048) (layer F.Cu) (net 8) (status 30))
 (segment (start 167.005 78.74) (end 170.815 78.74) (width 0.3048) (layer F.Cu) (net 8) (status 30))
 (segment (start 139.7 113.03) (end 140.97 111.76) (width 0.3048) (layer F.Cu) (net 8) (status 10))
 (segment (start 140.97 111.76) (end 140.97 109.855) (width 0.3048) (layer F.Cu) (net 8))
 (segment (start 137.769602 102.260398) (end 139.7 100.33) (width 0.3048) (layer F.Cu) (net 8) (status 20))
 (segment (start 137.769602 108.559602) (end 137.769602 102.260398) (width 0.3048) (layer F.Cu) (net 8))
 (segment (start 138.43 109.22) (end 137.769602 108.559602) (width 0.3048) (layer F.Cu) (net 8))
 (segment (start 140.335 109.22) (end 138.43 109.22) (width 0.3048) (layer F.Cu) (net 8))
 (segment (start 170.815 81.28) (end 167.005 81.28) (width 0.3048) (layer F.Cu) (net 11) (status 30))
 (segment (start 167.005 81.28) (end 156.845 81.28) (width 0.3048) (layer F.Cu) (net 11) (status 30)))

